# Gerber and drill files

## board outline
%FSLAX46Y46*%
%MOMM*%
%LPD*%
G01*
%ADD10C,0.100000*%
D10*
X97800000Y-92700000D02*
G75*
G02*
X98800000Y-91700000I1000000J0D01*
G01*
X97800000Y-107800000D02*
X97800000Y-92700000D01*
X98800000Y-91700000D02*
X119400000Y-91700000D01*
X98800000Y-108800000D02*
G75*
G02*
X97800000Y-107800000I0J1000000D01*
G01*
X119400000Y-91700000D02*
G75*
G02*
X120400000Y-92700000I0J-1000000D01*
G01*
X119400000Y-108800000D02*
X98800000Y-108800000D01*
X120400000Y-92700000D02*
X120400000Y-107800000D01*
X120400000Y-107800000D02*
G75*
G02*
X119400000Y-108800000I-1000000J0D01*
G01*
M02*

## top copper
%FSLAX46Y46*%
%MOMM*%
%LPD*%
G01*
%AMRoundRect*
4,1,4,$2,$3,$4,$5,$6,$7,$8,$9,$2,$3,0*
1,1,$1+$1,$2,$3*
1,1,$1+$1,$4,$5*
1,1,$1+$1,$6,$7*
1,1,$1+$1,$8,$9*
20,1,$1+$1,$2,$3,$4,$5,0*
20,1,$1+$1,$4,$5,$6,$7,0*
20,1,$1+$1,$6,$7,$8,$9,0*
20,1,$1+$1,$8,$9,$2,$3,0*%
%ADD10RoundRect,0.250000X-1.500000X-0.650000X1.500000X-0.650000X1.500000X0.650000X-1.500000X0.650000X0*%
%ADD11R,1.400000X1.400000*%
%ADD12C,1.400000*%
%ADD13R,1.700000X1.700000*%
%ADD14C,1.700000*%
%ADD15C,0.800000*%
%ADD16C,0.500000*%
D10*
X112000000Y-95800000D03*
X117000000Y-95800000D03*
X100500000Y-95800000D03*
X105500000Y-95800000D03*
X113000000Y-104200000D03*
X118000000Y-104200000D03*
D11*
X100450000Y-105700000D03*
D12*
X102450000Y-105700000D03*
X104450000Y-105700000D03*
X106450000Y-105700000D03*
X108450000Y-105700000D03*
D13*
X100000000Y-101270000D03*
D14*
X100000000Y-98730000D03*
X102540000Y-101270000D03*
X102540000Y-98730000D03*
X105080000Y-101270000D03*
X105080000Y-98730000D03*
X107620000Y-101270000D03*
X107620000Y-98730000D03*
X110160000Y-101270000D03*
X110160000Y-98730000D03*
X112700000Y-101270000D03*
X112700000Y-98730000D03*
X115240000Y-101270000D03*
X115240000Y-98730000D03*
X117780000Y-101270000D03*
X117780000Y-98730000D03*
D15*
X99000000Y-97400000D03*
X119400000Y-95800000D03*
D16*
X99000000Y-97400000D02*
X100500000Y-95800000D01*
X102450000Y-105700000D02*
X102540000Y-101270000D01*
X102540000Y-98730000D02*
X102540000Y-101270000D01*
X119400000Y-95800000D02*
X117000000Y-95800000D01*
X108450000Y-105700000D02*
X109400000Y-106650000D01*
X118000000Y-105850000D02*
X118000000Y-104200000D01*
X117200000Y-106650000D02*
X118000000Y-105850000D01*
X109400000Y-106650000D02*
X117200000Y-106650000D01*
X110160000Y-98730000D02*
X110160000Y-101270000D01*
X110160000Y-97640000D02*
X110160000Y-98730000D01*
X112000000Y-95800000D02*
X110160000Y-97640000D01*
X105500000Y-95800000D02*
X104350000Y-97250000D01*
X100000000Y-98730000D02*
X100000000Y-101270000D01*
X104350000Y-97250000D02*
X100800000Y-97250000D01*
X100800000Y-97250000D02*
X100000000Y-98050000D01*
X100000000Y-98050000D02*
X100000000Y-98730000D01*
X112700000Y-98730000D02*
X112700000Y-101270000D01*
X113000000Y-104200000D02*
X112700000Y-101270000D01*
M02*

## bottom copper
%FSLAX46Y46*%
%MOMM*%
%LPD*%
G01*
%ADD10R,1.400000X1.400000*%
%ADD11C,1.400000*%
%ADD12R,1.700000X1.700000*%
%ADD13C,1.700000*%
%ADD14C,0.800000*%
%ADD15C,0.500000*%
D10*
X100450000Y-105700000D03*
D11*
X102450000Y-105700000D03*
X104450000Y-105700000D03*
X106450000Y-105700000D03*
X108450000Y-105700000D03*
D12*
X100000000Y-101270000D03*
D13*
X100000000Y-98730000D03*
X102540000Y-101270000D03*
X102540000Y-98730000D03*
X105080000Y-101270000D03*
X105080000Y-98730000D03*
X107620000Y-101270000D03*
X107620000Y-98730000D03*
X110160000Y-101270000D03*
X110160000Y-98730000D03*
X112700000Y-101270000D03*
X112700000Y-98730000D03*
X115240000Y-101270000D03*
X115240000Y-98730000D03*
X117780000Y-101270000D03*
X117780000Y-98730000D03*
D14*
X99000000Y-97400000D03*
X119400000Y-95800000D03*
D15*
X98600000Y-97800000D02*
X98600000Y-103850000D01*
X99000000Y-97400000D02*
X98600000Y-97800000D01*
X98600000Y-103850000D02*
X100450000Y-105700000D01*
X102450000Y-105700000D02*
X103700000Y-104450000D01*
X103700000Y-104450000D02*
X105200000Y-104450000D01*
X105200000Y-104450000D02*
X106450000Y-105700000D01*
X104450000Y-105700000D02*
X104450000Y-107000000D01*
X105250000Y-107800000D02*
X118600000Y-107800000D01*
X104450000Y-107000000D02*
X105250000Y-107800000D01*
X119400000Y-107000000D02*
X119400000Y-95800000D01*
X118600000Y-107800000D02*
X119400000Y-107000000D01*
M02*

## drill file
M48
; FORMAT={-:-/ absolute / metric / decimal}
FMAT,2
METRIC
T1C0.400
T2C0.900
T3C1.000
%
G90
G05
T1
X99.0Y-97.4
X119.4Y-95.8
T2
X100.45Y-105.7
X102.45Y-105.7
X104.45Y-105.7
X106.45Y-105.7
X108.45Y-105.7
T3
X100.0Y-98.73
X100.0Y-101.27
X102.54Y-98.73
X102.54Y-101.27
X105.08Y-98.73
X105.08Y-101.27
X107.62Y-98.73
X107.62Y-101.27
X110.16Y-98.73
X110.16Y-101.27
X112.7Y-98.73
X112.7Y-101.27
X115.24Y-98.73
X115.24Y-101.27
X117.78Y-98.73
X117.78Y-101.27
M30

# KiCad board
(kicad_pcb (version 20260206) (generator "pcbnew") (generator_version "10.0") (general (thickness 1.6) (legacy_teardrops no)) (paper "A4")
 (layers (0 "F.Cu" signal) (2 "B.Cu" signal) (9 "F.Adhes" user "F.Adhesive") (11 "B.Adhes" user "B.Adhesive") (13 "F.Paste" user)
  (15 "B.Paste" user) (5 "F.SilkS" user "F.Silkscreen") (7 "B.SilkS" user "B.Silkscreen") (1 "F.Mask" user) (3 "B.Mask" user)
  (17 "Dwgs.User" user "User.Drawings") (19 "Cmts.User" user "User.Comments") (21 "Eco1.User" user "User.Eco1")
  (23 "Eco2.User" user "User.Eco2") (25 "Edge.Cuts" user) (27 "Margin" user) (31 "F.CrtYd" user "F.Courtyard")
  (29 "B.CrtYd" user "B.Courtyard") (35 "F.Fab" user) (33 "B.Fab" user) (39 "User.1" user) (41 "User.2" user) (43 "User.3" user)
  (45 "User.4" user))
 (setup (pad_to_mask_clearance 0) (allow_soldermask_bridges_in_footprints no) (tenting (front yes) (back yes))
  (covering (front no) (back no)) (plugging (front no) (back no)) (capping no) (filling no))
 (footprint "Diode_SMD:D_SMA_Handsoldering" (layer "F.Cu") (at 114.5 95.8)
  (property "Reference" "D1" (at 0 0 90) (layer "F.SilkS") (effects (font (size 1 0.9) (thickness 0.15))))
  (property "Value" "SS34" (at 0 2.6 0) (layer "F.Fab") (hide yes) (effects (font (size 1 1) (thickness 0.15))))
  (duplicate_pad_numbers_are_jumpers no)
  (pad "1" smd roundrect (at -2.5 0) (size 3.5 1.8) (layers "F.Cu" "F.Mask" "F.Paste") (roundrect_rratio 0.1388888889) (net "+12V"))
  (pad "2" smd roundrect (at 2.5 0) (size 3.5 1.8) (layers "F.Cu" "F.Mask" "F.Paste") (roundrect_rratio 0.1388888889) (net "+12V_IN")))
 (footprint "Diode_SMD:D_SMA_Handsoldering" (layer "F.Cu") (at 103 95.8)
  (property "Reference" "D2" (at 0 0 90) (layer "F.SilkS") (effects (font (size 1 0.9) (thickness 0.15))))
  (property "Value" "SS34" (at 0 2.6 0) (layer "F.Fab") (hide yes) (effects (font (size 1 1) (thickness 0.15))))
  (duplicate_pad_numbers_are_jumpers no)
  (pad "1" smd roundrect (at -2.5 0) (size 3.5 1.8) (layers "F.Cu" "F.Mask" "F.Paste") (roundrect_rratio 0.1388888889) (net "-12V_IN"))
  (pad "2" smd roundrect (at 2.5 0) (size 3.5 1.8) (layers "F.Cu" "F.Mask" "F.Paste") (roundrect_rratio 0.1388888889) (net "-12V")))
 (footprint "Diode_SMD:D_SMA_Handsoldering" (layer "F.Cu") (at 115.5 104.2)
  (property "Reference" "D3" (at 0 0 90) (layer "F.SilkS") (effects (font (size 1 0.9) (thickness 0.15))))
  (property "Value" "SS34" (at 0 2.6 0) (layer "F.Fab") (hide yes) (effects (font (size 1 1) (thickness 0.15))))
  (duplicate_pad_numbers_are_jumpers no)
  (pad "1" smd roundrect (at -2.5 0) (size 3.5 1.8) (layers "F.Cu" "F.Mask" "F.Paste") (roundrect_rratio 0.1388888889) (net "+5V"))
  (pad "2" smd roundrect (at 2.5 0) (size 3.5 1.8) (layers "F.Cu" "F.Mask" "F.Paste") (roundrect_rratio 0.1388888889) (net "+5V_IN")))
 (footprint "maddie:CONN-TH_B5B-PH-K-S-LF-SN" (layer "F.Cu") (at 104.45 105.7 180)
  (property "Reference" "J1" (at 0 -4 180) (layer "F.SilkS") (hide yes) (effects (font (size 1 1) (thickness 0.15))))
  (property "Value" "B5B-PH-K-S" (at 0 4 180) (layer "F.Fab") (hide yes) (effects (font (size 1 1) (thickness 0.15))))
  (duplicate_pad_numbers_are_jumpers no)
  (pad "1" thru_hole rect (at 4 0 180) (size 1.4 1.4) (drill 0.900024) (layers "*.Cu" "*.Mask") (remove_unused_layers no) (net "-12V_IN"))
  (pad "2" thru_hole circle (at 2 0 180) (size 1.4 1.4) (drill 0.900024) (layers "*.Cu" "*.Mask") (remove_unused_layers no) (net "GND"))
  (pad "3" thru_hole circle (at 0 0 180) (size 1.4 1.4) (drill 0.900024) (layers "*.Cu" "*.Mask") (remove_unused_layers no) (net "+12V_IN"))
  (pad "4" thru_hole circle (at -2 0 180) (size 1.4 1.4) (drill 0.900024) (layers "*.Cu" "*.Mask") (remove_unused_layers no) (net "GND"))
  (pad "5" thru_hole circle (at -4 0 180) (size 1.4 1.4) (drill 0.900024) (layers "*.Cu" "*.Mask") (remove_unused_layers no) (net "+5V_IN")))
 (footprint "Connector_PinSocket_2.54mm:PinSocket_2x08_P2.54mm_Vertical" (layer "B.Cu") (at 100 101.27 -90)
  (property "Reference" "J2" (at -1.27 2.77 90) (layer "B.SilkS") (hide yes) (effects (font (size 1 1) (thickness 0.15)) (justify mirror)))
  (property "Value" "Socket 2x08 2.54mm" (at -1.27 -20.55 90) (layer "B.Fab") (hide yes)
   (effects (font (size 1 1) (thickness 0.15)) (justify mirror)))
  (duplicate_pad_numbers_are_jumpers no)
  (pad "1" thru_hole rect (at 0 0 270) (size 1.7 1.7) (drill 1) (layers "*.Cu" "*.Mask") (remove_unused_layers no) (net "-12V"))
  (pad "2" thru_hole circle (at -2.54 0 270) (size 1.7 1.7) (drill 1) (layers "*.Cu" "*.Mask") (remove_unused_layers no) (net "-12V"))
  (pad "3" thru_hole circle (at 0 -2.54 270) (size 1.7 1.7) (drill 1) (layers "*.Cu" "*.Mask") (remove_unused_layers no) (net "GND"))
  (pad "4" thru_hole circle (at -2.54 -2.54 270) (size 1.7 1.7) (drill 1) (layers "*.Cu" "*.Mask") (remove_unused_layers no) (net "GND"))
  (pad "5" thru_hole circle (at 0 -5.08 270) (size 1.7 1.7) (drill 1) (layers "*.Cu" "*.Mask") (remove_unused_layers no)
   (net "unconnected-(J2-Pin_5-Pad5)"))
  (pad "6" thru_hole circle (at -2.54 -5.08 270) (size 1.7 1.7) (drill 1) (layers "*.Cu" "*.Mask") (remove_unused_layers no)
   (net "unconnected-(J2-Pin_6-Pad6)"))
  (pad "7" thru_hole circle (at 0 -7.62 270) (size 1.7 1.7) (drill 1) (layers "*.Cu" "*.Mask") (remove_unused_layers no)
   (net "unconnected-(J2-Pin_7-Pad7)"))
  (pad "8" thru_hole circle (at -2.54 -7.62 270) (size 1.7 1.7) (drill 1) (layers "*.Cu" "*.Mask") (remove_unused_layers no)
   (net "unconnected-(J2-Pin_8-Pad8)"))
  (pad "9" thru_hole circle (at 0 -10.16 270) (size 1.7 1.7) (drill 1) (layers "*.Cu" "*.Mask") (remove_unused_layers no) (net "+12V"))
  (pad "10" thru_hole circle (at -2.54 -10.16 270) (size 1.7 1.7) (drill 1) (layers "*.Cu" "*.Mask") (remove_unused_layers no) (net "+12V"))
  (pad "11" thru_hole circle (at 0 -12.7 270) (size 1.7 1.7) (drill 1) (layers "*.Cu" "*.Mask") (remove_unused_layers no) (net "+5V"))
  (pad "12" thru_hole circle (at -2.54 -12.7 270) (size 1.7 1.7) (drill 1) (layers "*.Cu" "*.Mask") (remove_unused_layers no) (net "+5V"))
  (pad "13" thru_hole circle (at 0 -15.24 270) (size 1.7 1.7) (drill 1) (layers "*.Cu" "*.Mask") (remove_unused_layers no)
   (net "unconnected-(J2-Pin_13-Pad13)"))
  (pad "14" thru_hole circle (at -2.54 -15.24 270) (size 1.7 1.7) (drill 1) (layers "*.Cu" "*.Mask") (remove_unused_layers no)
   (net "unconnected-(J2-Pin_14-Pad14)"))
  (pad "15" thru_hole circle (at 0 -17.78 270) (size 1.7 1.7) (drill 1) (layers "*.Cu" "*.Mask") (remove_unused_layers no)
   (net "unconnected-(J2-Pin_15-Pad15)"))
  (pad "16" thru_hole circle (at -2.54 -17.78 270) (size 1.7 1.7) (drill 1) (layers "*.Cu" "*.Mask") (remove_unused_layers no)
   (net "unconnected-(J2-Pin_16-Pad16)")))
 (gr_arc (start 97.8 92.7) (mid 98.09289 91.99289) (end 98.8 91.7) (stroke (width 0.1) (type default)) (layer "Edge.Cuts"))
 (gr_line (start 97.8 107.8) (end 97.8 92.7) (stroke (width 0.1) (type default)) (layer "Edge.Cuts"))
 (gr_line (start 98.8 91.7) (end 119.4 91.7) (stroke (width 0.1) (type default)) (layer "Edge.Cuts"))
 (gr_arc (start 98.8 108.8) (mid 98.09289 108.50711) (end 97.8 107.8) (stroke (width 0.1) (type default)) (layer "Edge.Cuts"))
 (gr_arc (start 119.4 91.7) (mid 120.10711 91.99289) (end 120.4 92.7) (stroke (width 0.1) (type default)) (layer "Edge.Cuts"))
 (gr_line (start 119.4 108.8) (end 98.8 108.8) (stroke (width 0.1) (type default)) (layer "Edge.Cuts"))
 (gr_line (start 120.4 92.7) (end 120.4 107.8) (stroke (width 0.1) (type default)) (layer "Edge.Cuts"))
 (gr_arc (start 120.4 107.8) (mid 120.10711 108.50711) (end 119.4 108.8) (stroke (width 0.1) (type default)) (layer "Edge.Cuts"))
 (segment (start 99 97.4) (end 100.5 95.8) (width 0.5) (layer "F.Cu") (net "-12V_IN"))
 (via (at 99 97.4) (size 0.8) (drill 0.4) (layers "F.Cu" "B.Cu") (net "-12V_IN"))
 (segment (start 98.6 97.8) (end 98.6 103.85) (width 0.5) (layer "B.Cu") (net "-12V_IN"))
 (segment (start 99 97.4) (end 98.6 97.8) (width 0.5) (layer "B.Cu") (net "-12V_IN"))
 (segment (start 98.6 103.85) (end 100.45 105.7) (width 0.5) (layer "B.Cu") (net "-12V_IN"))
 (segment (start 102.45 105.7) (end 102.54 101.27) (width 0.5) (layer "F.Cu") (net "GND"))
 (segment (start 102.54 98.73) (end 102.54 101.27) (width 0.5) (layer "F.Cu") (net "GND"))
 (segment (start 102.45 105.7) (end 103.7 104.45) (width 0.5) (layer "B.Cu") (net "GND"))
 (segment (start 103.7 104.45) (end 105.2 104.45) (width 0.5) (layer "B.Cu") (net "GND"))
 (segment (start 105.2 104.45) (end 106.45 105.7) (width 0.5) (layer "B.Cu") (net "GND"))
 (segment (start 119.4 95.8) (end 117 95.8) (width 0.5) (layer "F.Cu") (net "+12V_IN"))
 (via (at 119.4 95.8) (size 0.8) (drill 0.4) (layers "F.Cu" "B.Cu") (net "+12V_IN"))
 (segment (start 104.45 105.7) (end 104.45 107) (width 0.5) (layer "B.Cu") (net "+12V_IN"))
 (segment (start 105.25 107.8) (end 118.6 107.8) (width 0.5) (layer "B.Cu") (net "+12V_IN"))
 (segment (start 104.45 107) (end 105.25 107.8) (width 0.5) (layer "B.Cu") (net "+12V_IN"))
 (segment (start 119.4 107) (end 119.4 95.8) (width 0.5) (layer "B.Cu") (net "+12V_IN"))
 (segment (start 118.6 107.8) (end 119.4 107) (width 0.5) (layer "B.Cu") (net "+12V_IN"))
 (segment (start 108.45 105.7) (end 109.4 106.65) (width 0.5) (layer "F.Cu") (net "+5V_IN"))
 (segment (start 118 105.85) (end 118 104.2) (width 0.5) (layer "F.Cu") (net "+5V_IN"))
 (segment (start 117.2 106.65) (end 118 105.85) (width 0.5) (layer "F.Cu") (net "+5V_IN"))
 (segment (start 109.4 106.65) (end 117.2 106.65) (width 0.5) (layer "F.Cu") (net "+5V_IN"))
 (segment (start 110.16 98.73) (end 110.16 101.27) (width 0.5) (layer "F.Cu") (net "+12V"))
 (segment (start 110.16 97.64) (end 110.16 98.73) (width 0.5) (layer "F.Cu") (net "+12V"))
 (segment (start 112 95.8) (end 110.16 97.64) (width 0.5) (layer "F.Cu") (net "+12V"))
 (segment (start 105.5 95.8) (end 104.35 97.25) (width 0.5) (layer "F.Cu") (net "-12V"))
 (segment (start 100 98.73) (end 100 101.27) (width 0.5) (layer "F.Cu") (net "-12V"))
 (segment (start 104.35 97.25) (end 100.8 97.25) (width 0.5) (layer "F.Cu") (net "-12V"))
 (segment (start 100.8 97.25) (end 100 98.05) (width 0.5) (layer "F.Cu") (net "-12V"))
 (segment (start 100 98.05) (end 100 98.73) (width 0.5) (layer "F.Cu") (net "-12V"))
 (segment (start 112.7 98.73) (end 112.7 101.27) (width 0.5) (layer "F.Cu") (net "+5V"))
 (segment (start 113 104.2) (end 112.7 101.27) (width 0.5) (layer "F.Cu") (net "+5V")))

